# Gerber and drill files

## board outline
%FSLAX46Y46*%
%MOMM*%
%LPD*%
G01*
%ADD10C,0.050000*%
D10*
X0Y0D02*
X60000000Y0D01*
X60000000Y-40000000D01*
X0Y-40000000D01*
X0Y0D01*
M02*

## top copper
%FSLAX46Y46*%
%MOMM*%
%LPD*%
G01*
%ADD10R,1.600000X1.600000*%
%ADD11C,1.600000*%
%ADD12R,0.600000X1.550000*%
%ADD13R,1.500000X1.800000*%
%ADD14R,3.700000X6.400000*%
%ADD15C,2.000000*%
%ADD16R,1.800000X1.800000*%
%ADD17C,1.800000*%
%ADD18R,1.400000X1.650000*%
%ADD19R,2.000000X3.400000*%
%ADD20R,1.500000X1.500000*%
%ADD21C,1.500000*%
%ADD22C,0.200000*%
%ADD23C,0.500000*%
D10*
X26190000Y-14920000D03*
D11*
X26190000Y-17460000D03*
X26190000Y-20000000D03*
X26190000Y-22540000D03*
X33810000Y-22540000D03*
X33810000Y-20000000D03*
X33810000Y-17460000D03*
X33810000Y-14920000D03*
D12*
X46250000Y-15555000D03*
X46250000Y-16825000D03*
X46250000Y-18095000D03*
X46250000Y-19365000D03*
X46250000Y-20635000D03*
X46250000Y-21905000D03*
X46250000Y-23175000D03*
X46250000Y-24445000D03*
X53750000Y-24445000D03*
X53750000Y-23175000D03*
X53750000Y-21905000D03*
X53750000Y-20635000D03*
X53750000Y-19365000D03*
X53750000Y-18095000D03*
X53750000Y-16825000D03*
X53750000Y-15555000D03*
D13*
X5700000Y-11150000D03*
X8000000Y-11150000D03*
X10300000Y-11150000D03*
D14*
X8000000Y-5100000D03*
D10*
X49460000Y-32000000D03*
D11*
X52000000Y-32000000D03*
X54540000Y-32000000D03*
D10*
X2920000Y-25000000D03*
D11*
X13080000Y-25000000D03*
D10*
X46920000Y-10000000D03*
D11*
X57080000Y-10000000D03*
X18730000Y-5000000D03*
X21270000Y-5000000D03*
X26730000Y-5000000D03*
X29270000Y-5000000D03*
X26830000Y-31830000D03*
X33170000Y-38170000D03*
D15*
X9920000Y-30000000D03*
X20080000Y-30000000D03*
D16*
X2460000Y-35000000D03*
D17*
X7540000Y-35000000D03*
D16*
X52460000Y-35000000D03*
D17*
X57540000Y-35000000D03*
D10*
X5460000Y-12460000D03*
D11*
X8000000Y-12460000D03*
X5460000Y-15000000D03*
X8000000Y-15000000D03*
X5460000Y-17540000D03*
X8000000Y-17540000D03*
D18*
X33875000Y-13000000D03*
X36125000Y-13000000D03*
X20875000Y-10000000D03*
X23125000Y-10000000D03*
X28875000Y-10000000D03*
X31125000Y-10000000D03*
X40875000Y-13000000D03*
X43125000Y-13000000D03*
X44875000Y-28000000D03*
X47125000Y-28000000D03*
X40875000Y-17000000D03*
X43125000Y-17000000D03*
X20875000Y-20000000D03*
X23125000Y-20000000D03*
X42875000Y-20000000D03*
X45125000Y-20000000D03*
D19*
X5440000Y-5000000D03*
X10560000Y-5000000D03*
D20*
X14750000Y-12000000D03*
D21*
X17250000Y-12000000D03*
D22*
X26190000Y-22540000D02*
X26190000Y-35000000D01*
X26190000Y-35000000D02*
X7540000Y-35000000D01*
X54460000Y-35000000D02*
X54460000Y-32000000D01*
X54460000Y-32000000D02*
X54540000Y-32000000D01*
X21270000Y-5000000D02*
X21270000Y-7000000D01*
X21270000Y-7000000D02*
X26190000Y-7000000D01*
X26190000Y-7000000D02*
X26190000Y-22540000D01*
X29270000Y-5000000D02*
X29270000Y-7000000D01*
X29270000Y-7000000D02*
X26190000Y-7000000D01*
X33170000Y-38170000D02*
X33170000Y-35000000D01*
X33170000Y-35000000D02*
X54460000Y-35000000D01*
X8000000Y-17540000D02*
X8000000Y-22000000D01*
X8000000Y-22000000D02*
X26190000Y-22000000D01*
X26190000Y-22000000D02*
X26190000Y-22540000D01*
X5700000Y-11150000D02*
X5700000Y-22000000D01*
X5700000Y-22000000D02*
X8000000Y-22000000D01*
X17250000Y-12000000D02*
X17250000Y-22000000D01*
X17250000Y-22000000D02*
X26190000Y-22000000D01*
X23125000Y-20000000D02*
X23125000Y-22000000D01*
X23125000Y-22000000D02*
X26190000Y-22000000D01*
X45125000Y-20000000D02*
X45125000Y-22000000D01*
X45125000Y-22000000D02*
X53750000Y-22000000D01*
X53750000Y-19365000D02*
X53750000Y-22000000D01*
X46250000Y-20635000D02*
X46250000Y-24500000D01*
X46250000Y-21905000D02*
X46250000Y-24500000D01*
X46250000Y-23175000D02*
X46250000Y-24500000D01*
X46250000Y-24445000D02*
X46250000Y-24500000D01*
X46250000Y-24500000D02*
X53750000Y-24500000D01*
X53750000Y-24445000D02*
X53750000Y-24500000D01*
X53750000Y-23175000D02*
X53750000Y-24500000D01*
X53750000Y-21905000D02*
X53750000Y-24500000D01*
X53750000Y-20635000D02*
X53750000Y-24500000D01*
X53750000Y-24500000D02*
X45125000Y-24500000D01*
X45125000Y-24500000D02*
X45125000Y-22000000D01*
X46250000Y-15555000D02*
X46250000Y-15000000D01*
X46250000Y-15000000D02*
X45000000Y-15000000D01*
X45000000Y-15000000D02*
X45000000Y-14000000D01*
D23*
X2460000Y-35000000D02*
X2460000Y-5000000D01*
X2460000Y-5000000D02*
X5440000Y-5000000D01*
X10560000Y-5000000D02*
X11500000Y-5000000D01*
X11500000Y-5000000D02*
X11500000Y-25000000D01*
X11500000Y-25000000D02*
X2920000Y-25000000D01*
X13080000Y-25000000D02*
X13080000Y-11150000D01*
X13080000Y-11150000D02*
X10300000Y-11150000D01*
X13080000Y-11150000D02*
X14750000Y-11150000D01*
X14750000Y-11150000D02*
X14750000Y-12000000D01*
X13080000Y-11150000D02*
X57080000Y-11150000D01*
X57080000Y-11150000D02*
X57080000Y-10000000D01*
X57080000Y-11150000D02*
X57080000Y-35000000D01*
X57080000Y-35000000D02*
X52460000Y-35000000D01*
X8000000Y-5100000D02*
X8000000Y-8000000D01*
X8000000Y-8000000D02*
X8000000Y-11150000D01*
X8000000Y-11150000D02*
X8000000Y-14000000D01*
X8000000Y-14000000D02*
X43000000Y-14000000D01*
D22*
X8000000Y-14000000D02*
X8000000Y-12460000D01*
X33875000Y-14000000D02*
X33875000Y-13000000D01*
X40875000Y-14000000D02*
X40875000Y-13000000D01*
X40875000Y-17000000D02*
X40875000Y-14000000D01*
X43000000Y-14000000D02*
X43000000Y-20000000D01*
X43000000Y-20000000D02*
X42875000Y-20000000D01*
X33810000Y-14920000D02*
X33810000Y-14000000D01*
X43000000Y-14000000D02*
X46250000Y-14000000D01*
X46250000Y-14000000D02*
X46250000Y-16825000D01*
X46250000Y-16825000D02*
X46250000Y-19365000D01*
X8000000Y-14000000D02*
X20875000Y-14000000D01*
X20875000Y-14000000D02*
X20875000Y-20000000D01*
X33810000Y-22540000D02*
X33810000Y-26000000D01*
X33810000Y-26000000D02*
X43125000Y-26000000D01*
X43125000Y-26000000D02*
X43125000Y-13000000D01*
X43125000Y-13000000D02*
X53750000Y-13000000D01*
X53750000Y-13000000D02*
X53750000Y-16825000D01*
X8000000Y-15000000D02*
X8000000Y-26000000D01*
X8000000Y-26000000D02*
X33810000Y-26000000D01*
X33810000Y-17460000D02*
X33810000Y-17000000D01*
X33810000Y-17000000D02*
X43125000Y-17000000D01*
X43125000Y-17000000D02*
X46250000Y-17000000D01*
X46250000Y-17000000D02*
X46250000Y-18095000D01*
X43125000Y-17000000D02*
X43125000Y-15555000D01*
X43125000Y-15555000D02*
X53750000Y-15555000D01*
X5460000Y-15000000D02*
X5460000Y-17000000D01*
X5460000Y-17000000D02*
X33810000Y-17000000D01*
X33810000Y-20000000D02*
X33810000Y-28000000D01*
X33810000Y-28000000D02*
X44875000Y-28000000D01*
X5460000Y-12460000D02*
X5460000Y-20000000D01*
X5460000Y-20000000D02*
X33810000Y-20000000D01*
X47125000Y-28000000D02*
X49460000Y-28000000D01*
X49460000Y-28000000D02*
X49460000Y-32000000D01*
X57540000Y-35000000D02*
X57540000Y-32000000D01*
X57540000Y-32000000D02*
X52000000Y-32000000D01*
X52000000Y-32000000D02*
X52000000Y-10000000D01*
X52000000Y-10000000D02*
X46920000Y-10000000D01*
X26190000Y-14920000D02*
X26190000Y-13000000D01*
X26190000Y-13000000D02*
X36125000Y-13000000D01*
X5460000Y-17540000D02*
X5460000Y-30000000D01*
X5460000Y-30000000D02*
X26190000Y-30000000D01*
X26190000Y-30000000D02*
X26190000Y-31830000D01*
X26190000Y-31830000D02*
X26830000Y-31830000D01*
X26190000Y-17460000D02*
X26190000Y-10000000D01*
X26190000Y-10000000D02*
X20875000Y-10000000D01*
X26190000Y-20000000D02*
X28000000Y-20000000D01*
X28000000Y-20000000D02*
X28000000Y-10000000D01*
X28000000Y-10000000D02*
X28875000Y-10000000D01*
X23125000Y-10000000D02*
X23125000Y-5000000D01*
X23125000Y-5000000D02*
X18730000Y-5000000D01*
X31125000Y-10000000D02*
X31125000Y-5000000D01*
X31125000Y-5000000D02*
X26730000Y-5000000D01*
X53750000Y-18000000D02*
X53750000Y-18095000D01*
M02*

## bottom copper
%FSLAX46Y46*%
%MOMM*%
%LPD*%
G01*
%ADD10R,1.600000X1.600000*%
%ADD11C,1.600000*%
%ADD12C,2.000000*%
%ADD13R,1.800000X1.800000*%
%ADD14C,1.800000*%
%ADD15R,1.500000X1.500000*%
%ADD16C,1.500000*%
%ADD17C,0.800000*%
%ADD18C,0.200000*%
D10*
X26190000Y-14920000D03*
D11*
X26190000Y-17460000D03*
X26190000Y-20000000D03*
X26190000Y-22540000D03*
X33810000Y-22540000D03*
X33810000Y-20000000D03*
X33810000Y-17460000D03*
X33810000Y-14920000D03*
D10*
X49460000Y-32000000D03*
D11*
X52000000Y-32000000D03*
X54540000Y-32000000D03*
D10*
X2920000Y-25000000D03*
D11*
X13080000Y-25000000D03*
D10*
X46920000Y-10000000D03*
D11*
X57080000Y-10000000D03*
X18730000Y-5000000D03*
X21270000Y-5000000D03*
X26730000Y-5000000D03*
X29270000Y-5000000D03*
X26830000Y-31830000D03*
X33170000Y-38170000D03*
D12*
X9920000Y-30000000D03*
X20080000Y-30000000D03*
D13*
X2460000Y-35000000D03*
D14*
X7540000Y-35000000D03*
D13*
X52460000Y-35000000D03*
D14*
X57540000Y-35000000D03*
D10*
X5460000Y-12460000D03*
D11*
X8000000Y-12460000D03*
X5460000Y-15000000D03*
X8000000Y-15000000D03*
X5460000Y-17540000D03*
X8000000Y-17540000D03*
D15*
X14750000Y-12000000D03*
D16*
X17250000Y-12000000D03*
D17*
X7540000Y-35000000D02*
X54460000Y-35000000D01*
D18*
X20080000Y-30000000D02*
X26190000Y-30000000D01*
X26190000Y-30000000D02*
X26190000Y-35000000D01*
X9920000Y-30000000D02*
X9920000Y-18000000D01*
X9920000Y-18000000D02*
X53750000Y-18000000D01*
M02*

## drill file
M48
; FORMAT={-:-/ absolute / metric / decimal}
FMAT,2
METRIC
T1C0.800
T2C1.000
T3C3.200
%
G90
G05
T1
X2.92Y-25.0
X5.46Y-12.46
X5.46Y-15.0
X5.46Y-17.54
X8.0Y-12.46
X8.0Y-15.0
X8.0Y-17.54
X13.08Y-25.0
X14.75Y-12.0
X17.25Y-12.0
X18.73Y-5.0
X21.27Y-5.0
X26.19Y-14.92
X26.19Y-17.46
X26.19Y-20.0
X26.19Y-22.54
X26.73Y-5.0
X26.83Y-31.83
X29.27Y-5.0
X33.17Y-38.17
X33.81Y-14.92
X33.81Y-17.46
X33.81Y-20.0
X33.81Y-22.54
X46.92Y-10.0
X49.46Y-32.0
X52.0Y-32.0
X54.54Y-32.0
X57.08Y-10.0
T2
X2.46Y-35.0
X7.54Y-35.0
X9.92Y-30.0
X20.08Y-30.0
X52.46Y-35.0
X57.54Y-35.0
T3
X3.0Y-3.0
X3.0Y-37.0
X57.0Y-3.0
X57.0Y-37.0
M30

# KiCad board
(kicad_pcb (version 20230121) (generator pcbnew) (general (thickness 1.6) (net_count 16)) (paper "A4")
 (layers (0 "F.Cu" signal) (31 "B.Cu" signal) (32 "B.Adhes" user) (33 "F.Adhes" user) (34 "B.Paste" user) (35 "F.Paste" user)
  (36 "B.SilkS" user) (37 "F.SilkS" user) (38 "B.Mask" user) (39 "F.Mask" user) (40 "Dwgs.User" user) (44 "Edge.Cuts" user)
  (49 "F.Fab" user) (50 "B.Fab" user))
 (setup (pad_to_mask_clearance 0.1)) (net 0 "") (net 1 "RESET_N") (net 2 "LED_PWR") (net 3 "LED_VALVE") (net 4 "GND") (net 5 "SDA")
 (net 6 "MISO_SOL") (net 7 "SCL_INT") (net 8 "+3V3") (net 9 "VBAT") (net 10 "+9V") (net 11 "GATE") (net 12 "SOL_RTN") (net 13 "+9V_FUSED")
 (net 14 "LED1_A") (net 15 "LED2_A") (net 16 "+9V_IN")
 (gr_rect (start 0 0) (end 60 40) (stroke (width 0.05) (type solid)) (layer "Edge.Cuts"))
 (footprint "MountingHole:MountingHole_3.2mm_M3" (layer "F.Cu") (at 3 3) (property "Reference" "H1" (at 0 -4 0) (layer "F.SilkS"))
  (pad "" np_thru_hole circle (at 0 0) (size 3.2 3.2) (drill 3.2) (layers "*.Cu" "*.Mask")))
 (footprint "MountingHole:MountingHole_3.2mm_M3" (layer "F.Cu") (at 57 3) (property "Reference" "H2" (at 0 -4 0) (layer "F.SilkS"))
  (pad "" np_thru_hole circle (at 0 0) (size 3.2 3.2) (drill 3.2) (layers "*.Cu" "*.Mask")))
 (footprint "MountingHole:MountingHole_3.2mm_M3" (layer "F.Cu") (at 3 37) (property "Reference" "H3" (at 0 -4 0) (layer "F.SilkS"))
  (pad "" np_thru_hole circle (at 0 0) (size 3.2 3.2) (drill 3.2) (layers "*.Cu" "*.Mask")))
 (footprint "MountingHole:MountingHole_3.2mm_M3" (layer "F.Cu") (at 57 37) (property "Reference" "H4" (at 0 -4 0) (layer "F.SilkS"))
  (pad "" np_thru_hole circle (at 0 0) (size 3.2 3.2) (drill 3.2) (layers "*.Cu" "*.Mask")))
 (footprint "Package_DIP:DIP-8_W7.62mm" (layer "F.Cu") (at 30 20) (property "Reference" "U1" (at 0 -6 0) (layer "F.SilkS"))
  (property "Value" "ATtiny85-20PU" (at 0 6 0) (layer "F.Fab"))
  (pad "1" thru_hole rect (at -3.8100 -5.0800) (size 1.6 1.6) (drill 0.8) (layers "*.Cu" "*.Mask") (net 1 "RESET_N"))
  (pad "2" thru_hole circle (at -3.8100 -2.5400) (size 1.6 1.6) (drill 0.8) (layers "*.Cu" "*.Mask") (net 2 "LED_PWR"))
  (pad "3" thru_hole circle (at -3.8100 0.0000) (size 1.6 1.6) (drill 0.8) (layers "*.Cu" "*.Mask") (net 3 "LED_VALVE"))
  (pad "4" thru_hole circle (at -3.8100 2.5400) (size 1.6 1.6) (drill 0.8) (layers "*.Cu" "*.Mask") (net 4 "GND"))
  (pad "5" thru_hole circle (at 3.8100 2.5400) (size 1.6 1.6) (drill 0.8) (layers "*.Cu" "*.Mask") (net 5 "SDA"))
  (pad "6" thru_hole circle (at 3.8100 0.0000) (size 1.6 1.6) (drill 0.8) (layers "*.Cu" "*.Mask") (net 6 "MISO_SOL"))
  (pad "7" thru_hole circle (at 3.8100 -2.5400) (size 1.6 1.6) (drill 0.8) (layers "*.Cu" "*.Mask") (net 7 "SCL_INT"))
  (pad "8" thru_hole circle (at 3.8100 -5.0800) (size 1.6 1.6) (drill 0.8) (layers "*.Cu" "*.Mask") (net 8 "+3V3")))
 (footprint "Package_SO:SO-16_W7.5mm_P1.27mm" (layer "F.Cu") (at 50 20) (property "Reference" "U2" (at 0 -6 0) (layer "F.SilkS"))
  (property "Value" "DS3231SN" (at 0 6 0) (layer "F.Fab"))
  (pad "1" smd rect (at -3.75 -4.4450) (size 0.6 1.55) (layers "F.Cu" "F.Paste" "F.Mask") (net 4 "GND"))
  (pad "2" smd rect (at -3.75 -3.1750) (size 0.6 1.55) (layers "F.Cu" "F.Paste" "F.Mask") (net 8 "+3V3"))
  (pad "3" smd rect (at -3.75 -1.9050) (size 0.6 1.55) (layers "F.Cu" "F.Paste" "F.Mask") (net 7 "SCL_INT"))
  (pad "4" smd rect (at -3.75 -0.6350) (size 0.6 1.55) (layers "F.Cu" "F.Paste" "F.Mask") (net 8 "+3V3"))
  (pad "5" smd rect (at -3.75 0.6350) (size 0.6 1.55) (layers "F.Cu" "F.Paste" "F.Mask") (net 4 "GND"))
  (pad "6" smd rect (at -3.75 1.9050) (size 0.6 1.55) (layers "F.Cu" "F.Paste" "F.Mask") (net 4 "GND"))
  (pad "7" smd rect (at -3.75 3.1750) (size 0.6 1.55) (layers "F.Cu" "F.Paste" "F.Mask") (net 4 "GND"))
  (pad "8" smd rect (at -3.75 4.4450) (size 0.6 1.55) (layers "F.Cu" "F.Paste" "F.Mask") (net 4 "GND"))
  (pad "9" smd rect (at 3.75 4.4450) (size 0.6 1.55) (layers "F.Cu" "F.Paste" "F.Mask") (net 4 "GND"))
  (pad "10" smd rect (at 3.75 3.1750) (size 0.6 1.55) (layers "F.Cu" "F.Paste" "F.Mask") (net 4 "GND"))
  (pad "11" smd rect (at 3.75 1.9050) (size 0.6 1.55) (layers "F.Cu" "F.Paste" "F.Mask") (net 4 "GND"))
  (pad "12" smd rect (at 3.75 0.6350) (size 0.6 1.55) (layers "F.Cu" "F.Paste" "F.Mask") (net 4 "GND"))
  (pad "13" smd rect (at 3.75 -0.6350) (size 0.6 1.55) (layers "F.Cu" "F.Paste" "F.Mask") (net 4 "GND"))
  (pad "14" smd rect (at 3.75 -1.9050) (size 0.6 1.55) (layers "F.Cu" "F.Paste" "F.Mask") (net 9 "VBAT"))
  (pad "15" smd rect (at 3.75 -3.1750) (size 0.6 1.55) (layers "F.Cu" "F.Paste" "F.Mask") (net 5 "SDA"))
  (pad "16" smd rect (at 3.75 -4.4450) (size 0.6 1.55) (layers "F.Cu" "F.Paste" "F.Mask") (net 7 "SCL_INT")))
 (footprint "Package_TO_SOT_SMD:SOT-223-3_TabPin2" (layer "F.Cu") (at 8 8) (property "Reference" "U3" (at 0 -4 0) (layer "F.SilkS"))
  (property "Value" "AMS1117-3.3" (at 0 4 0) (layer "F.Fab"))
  (pad "1" smd rect (at -2.3000 3.1500) (size 1.5 1.8) (layers "F.Cu" "F.Paste" "F.Mask") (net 4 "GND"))
  (pad "2" smd rect (at 0.0000 3.1500) (size 1.5 1.8) (layers "F.Cu" "F.Paste" "F.Mask") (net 8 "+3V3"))
  (pad "3" smd rect (at 2.3000 3.1500) (size 1.5 1.8) (layers "F.Cu" "F.Paste" "F.Mask") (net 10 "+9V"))
  (pad "4" smd rect (at 0 -2.9) (size 3.7 6.4) (layers "F.Cu" "F.Paste" "F.Mask") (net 8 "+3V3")))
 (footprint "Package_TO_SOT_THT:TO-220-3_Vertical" (layer "F.Cu") (at 52 32) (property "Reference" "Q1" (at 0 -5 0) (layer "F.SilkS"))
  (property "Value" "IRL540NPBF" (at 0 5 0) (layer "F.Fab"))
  (pad "1" thru_hole rect (at -2.5400 0) (size 1.6 1.6) (drill 0.8) (layers "*.Cu" "*.Mask") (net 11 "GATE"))
  (pad "2" thru_hole circle (at 0.0000 0) (size 1.6 1.6) (drill 0.8) (layers "*.Cu" "*.Mask") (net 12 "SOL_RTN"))
  (pad "3" thru_hole circle (at 2.5400 0) (size 1.6 1.6) (drill 0.8) (layers "*.Cu" "*.Mask") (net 4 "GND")))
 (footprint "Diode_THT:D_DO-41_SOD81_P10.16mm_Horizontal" (layer "F.Cu") (at 8 25) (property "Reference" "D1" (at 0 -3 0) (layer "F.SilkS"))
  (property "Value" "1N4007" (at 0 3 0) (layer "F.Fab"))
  (pad "A" thru_hole rect (at -5.0800 0) (size 1.6 1.6) (drill 0.8) (layers "*.Cu" "*.Mask") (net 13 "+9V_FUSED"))
  (pad "K" thru_hole circle (at 5.0800 0) (size 1.6 1.6) (drill 0.8) (layers "*.Cu" "*.Mask") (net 10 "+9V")))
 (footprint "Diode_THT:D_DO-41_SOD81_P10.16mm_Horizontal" (layer "F.Cu") (at 52 10)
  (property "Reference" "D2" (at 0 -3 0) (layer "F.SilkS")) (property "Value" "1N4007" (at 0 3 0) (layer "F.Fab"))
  (pad "A" thru_hole rect (at -5.0800 0) (size 1.6 1.6) (drill 0.8) (layers "*.Cu" "*.Mask") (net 12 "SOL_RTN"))
  (pad "K" thru_hole circle (at 5.0800 0) (size 1.6 1.6) (drill 0.8) (layers "*.Cu" "*.Mask") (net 10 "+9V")))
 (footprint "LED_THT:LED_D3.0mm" (layer "F.Cu") (at 20 5) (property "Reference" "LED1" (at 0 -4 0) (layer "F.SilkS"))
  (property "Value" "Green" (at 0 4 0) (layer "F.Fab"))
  (pad "A" thru_hole circle (at -1.2700 0) (size 1.6 1.6) (drill 0.8) (layers "*.Cu" "*.Mask") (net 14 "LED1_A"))
  (pad "K" thru_hole circle (at 1.2700 0) (size 1.6 1.6) (drill 0.8) (layers "*.Cu" "*.Mask") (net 4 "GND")))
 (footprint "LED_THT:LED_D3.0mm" (layer "F.Cu") (at 28 5) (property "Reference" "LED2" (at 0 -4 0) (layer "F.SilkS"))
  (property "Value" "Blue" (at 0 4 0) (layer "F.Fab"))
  (pad "A" thru_hole circle (at -1.2700 0) (size 1.6 1.6) (drill 0.8) (layers "*.Cu" "*.Mask") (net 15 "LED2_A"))
  (pad "K" thru_hole circle (at 1.2700 0) (size 1.6 1.6) (drill 0.8) (layers "*.Cu" "*.Mask") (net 4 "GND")))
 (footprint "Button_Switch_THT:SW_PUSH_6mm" (layer "F.Cu") (at 30 35) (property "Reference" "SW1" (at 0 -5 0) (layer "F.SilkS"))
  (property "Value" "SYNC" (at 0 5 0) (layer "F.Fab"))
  (pad "1" thru_hole circle (at -3.1700 -3.1700) (size 1.6 1.6) (drill 0.8) (layers "*.Cu" "*.Mask") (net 1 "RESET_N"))
  (pad "2" thru_hole circle (at 3.1700 3.1700) (size 1.6 1.6) (drill 0.8) (layers "*.Cu" "*.Mask") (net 4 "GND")))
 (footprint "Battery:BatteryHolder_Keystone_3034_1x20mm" (layer "B.Cu") (at 15 30)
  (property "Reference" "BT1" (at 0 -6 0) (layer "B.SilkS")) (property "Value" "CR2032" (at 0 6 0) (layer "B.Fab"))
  (pad "+" thru_hole circle (at -5.0800 0) (size 2 2) (drill 1) (layers "*.Cu" "*.Mask") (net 9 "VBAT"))
  (pad "-" thru_hole circle (at 5.0800 0) (size 2 2) (drill 1) (layers "*.Cu" "*.Mask") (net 4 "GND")))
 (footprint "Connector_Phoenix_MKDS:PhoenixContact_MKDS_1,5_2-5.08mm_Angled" (layer "F.Cu") (at 5 35)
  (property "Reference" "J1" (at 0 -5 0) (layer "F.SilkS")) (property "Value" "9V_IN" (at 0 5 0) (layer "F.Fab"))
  (pad "1" thru_hole rect (at -2.5400 0) (size 1.8 1.8) (drill 1) (layers "*.Cu" "*.Mask") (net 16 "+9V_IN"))
  (pad "2" thru_hole circle (at 2.5400 0) (size 1.8 1.8) (drill 1) (layers "*.Cu" "*.Mask") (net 4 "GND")))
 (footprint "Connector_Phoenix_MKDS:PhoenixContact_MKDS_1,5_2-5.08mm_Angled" (layer "F.Cu") (at 55 35)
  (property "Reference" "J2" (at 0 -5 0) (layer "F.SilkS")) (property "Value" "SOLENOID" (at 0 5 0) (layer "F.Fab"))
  (pad "1" thru_hole rect (at -2.5400 0) (size 1.8 1.8) (drill 1) (layers "*.Cu" "*.Mask") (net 10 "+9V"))
  (pad "2" thru_hole circle (at 2.5400 0) (size 1.8 1.8) (drill 1) (layers "*.Cu" "*.Mask") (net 12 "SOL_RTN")))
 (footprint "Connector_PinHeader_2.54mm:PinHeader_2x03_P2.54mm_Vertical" (layer "F.Cu") (at 8 15)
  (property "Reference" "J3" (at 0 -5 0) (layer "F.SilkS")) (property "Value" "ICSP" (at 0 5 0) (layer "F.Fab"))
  (pad "1" thru_hole rect (at -2.5400 -2.5400) (size 1.6 1.6) (drill 0.8) (layers "*.Cu" "*.Mask") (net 6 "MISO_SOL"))
  (pad "2" thru_hole circle (at 0.0000 -2.5400) (size 1.6 1.6) (drill 0.8) (layers "*.Cu" "*.Mask") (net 8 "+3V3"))
  (pad "3" thru_hole circle (at -2.5400 0.0000) (size 1.6 1.6) (drill 0.8) (layers "*.Cu" "*.Mask") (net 7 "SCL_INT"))
  (pad "4" thru_hole circle (at 0.0000 0.0000) (size 1.6 1.6) (drill 0.8) (layers "*.Cu" "*.Mask") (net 5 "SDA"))
  (pad "5" thru_hole circle (at -2.5400 2.5400) (size 1.6 1.6) (drill 0.8) (layers "*.Cu" "*.Mask") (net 1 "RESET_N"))
  (pad "6" thru_hole circle (at 0.0000 2.5400) (size 1.6 1.6) (drill 0.8) (layers "*.Cu" "*.Mask") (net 4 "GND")))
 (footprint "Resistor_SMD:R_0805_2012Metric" (layer "F.Cu") (at 35 13) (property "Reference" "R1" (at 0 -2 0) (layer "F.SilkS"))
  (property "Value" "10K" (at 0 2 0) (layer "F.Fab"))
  (pad "1" smd rect (at -1.1250 0) (size 1.4 1.65) (layers "F.Cu" "F.Paste" "F.Mask") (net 8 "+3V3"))
  (pad "2" smd rect (at 1.1250 0) (size 1.4 1.65) (layers "F.Cu" "F.Paste" "F.Mask") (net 1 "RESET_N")))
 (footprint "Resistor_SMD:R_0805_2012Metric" (layer "F.Cu") (at 22 10) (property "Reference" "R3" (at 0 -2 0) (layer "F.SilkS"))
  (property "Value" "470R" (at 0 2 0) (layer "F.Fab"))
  (pad "1" smd rect (at -1.1250 0) (size 1.4 1.65) (layers "F.Cu" "F.Paste" "F.Mask") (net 2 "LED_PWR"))
  (pad "2" smd rect (at 1.1250 0) (size 1.4 1.65) (layers "F.Cu" "F.Paste" "F.Mask") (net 14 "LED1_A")))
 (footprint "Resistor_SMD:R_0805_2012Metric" (layer "F.Cu") (at 30 10) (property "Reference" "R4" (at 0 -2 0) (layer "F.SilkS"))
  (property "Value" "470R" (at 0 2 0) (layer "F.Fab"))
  (pad "1" smd rect (at -1.1250 0) (size 1.4 1.65) (layers "F.Cu" "F.Paste" "F.Mask") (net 3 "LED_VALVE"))
  (pad "2" smd rect (at 1.1250 0) (size 1.4 1.65) (layers "F.Cu" "F.Paste" "F.Mask") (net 15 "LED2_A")))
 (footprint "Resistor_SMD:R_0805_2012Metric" (layer "F.Cu") (at 42 13) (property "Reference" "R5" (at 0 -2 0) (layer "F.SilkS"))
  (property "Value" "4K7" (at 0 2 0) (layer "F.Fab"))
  (pad "1" smd rect (at -1.1250 0) (size 1.4 1.65) (layers "F.Cu" "F.Paste" "F.Mask") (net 8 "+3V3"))
  (pad "2" smd rect (at 1.1250 0) (size 1.4 1.65) (layers "F.Cu" "F.Paste" "F.Mask") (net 5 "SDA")))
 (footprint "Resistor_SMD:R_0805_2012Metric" (layer "F.Cu") (at 46 28) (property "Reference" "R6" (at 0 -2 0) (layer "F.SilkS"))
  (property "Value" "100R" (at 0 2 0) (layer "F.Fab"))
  (pad "1" smd rect (at -1.1250 0) (size 1.4 1.65) (layers "F.Cu" "F.Paste" "F.Mask") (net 6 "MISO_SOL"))
  (pad "2" smd rect (at 1.1250 0) (size 1.4 1.65) (layers "F.Cu" "F.Paste" "F.Mask") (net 11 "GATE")))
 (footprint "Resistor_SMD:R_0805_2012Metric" (layer "F.Cu") (at 42 17) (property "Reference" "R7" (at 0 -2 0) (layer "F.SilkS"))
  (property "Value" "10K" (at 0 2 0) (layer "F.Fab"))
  (pad "1" smd rect (at -1.1250 0) (size 1.4 1.65) (layers "F.Cu" "F.Paste" "F.Mask") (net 8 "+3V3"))
  (pad "2" smd rect (at 1.1250 0) (size 1.4 1.65) (layers "F.Cu" "F.Paste" "F.Mask") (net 7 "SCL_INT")))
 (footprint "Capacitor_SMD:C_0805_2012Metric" (layer "F.Cu") (at 22 20) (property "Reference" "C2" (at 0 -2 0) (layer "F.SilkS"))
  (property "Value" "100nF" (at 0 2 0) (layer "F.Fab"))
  (pad "1" smd rect (at -1.1250 0) (size 1.4 1.65) (layers "F.Cu" "F.Paste" "F.Mask") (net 8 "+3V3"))
  (pad "2" smd rect (at 1.1250 0) (size 1.4 1.65) (layers "F.Cu" "F.Paste" "F.Mask") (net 4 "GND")))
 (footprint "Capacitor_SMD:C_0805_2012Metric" (layer "F.Cu") (at 44 20) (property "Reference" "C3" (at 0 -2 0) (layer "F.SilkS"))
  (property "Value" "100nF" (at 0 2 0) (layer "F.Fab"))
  (pad "1" smd rect (at -1.1250 0) (size 1.4 1.65) (layers "F.Cu" "F.Paste" "F.Mask") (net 8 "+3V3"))
  (pad "2" smd rect (at 1.1250 0) (size 1.4 1.65) (layers "F.Cu" "F.Paste" "F.Mask") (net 4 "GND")))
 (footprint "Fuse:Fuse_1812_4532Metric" (layer "F.Cu") (at 8 5) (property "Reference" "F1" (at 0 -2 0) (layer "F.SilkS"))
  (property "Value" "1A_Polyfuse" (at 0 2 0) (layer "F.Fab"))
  (pad "1" smd rect (at -2.5600 0) (size 2.0 3.4) (layers "F.Cu" "F.Paste" "F.Mask") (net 16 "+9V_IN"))
  (pad "2" smd rect (at 2.5600 0) (size 2.0 3.4) (layers "F.Cu" "F.Paste" "F.Mask") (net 13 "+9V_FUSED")))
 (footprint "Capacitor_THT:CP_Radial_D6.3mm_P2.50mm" (layer "F.Cu") (at 16 12) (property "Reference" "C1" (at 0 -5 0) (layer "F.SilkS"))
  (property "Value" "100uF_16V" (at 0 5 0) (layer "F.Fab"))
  (pad "1" thru_hole rect (at -1.2500 0) (size 1.5 1.5) (drill 0.8) (layers "*.Cu" "*.Mask") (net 10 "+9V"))
  (pad "2" thru_hole circle (at 1.2500 0) (size 1.5 1.5) (drill 0.8) (layers "*.Cu" "*.Mask") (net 4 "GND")))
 (segment (start 7.5400 35.0000) (end 54.4600 35.0000) (width 0.8) (layer "B.Cu") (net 4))
 (segment (start 26.1900 22.5400) (end 26.1900 35.0000) (width 0.2) (layer "F.Cu") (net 4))
 (segment (start 26.1900 35.0000) (end 7.5400 35.0000) (width 0.2) (layer "F.Cu") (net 4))
 (segment (start 54.4600 35.0000) (end 54.4600 32.0000) (width 0.2) (layer "F.Cu") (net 4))
 (segment (start 54.4600 32.0000) (end 54.5400 32.0000) (width 0.2) (layer "F.Cu") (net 4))
 (segment (start 21.2700 5.0000) (end 21.2700 7.0000) (width 0.2) (layer "F.Cu") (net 4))
 (segment (start 21.2700 7.0000) (end 26.1900 7.0000) (width 0.2) (layer "F.Cu") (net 4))
 (segment (start 26.1900 7.0000) (end 26.1900 22.5400) (width 0.2) (layer "F.Cu") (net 4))
 (segment (start 29.2700 5.0000) (end 29.2700 7.0000) (width 0.2) (layer "F.Cu") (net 4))
 (segment (start 29.2700 7.0000) (end 26.1900 7.0000) (width 0.2) (layer "F.Cu") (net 4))
 (segment (start 33.1700 38.1700) (end 33.1700 35.0000) (width 0.2) (layer "F.Cu") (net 4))
 (segment (start 33.1700 35.0000) (end 54.4600 35.0000) (width 0.2) (layer "F.Cu") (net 4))
 (segment (start 8.0000 17.5400) (end 8.0000 22.0000) (width 0.2) (layer "F.Cu") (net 4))
 (segment (start 8.0000 22.0000) (end 26.1900 22.0000) (width 0.2) (layer "F.Cu") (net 4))
 (segment (start 26.1900 22.0000) (end 26.1900 22.5400) (width 0.2) (layer "F.Cu") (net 4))
 (segment (start 5.7000 11.1500) (end 5.7000 22.0000) (width 0.2) (layer "F.Cu") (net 4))
 (segment (start 5.7000 22.0000) (end 8.0000 22.0000) (width 0.2) (layer "F.Cu") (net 4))
 (segment (start 17.2500 12.0000) (end 17.2500 22.0000) (width 0.2) (layer "F.Cu") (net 4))
 (segment (start 17.2500 22.0000) (end 26.1900 22.0000) (width 0.2) (layer "F.Cu") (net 4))
 (segment (start 23.1250 20.0000) (end 23.1250 22.0000) (width 0.2) (layer "F.Cu") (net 4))
 (segment (start 23.1250 22.0000) (end 26.1900 22.0000) (width 0.2) (layer "F.Cu") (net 4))
 (segment (start 45.1250 20.0000) (end 45.1250 22.0000) (width 0.2) (layer "F.Cu") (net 4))
 (segment (start 45.1250 22.0000) (end 53.7500 22.0000) (width 0.2) (layer "F.Cu") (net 4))
 (segment (start 53.7500 19.3650) (end 53.7500 22.0000) (width 0.2) (layer "F.Cu") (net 4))
 (segment (start 46.2500 20.6350) (end 46.2500 24.5000) (width 0.2) (layer "F.Cu") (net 4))
 (segment (start 46.2500 21.9050) (end 46.2500 24.5000) (width 0.2) (layer "F.Cu") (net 4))
 (segment (start 46.2500 23.1750) (end 46.2500 24.5000) (width 0.2) (layer "F.Cu") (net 4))
 (segment (start 46.2500 24.4450) (end 46.2500 24.5000) (width 0.2) (layer "F.Cu") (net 4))
 (segment (start 46.2500 24.5000) (end 53.7500 24.5000) (width 0.2) (layer "F.Cu") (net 4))
 (segment (start 53.7500 24.4450) (end 53.7500 24.5000) (width 0.2) (layer "F.Cu") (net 4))
 (segment (start 53.7500 23.1750) (end 53.7500 24.5000) (width 0.2) (layer "F.Cu") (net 4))
 (segment (start 53.7500 21.9050) (end 53.7500 24.5000) (width 0.2) (layer "F.Cu") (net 4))
 (segment (start 53.7500 20.6350) (end 53.7500 24.5000) (width 0.2) (layer "F.Cu") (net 4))
 (segment (start 53.7500 24.5000) (end 45.1250 24.5000) (width 0.2) (layer "F.Cu") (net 4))
 (segment (start 45.1250 24.5000) (end 45.1250 22.0000) (width 0.2) (layer "F.Cu") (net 4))
 (segment (start 46.2500 15.5550) (end 46.2500 15.0000) (width 0.2) (layer "F.Cu") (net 4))
 (segment (start 46.2500 15.0000) (end 45.0000 15.0000) (width 0.2) (layer "F.Cu") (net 4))
 (segment (start 45.0000 15.0000) (end 45.0000 14.0000) (width 0.2) (layer "F.Cu") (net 4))
 (segment (start 20.0800 30.0000) (end 26.1900 30.0000) (width 0.2) (layer "B.Cu") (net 4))
 (segment (start 26.1900 30.0000) (end 26.1900 35.0000) (width 0.2) (layer "B.Cu") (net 4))
 (segment (start 2.4600 35.0000) (end 2.4600 5.0000) (width 0.5) (layer "F.Cu") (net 16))
 (segment (start 2.4600 5.0000) (end 5.4400 5.0000) (width 0.5) (layer "F.Cu") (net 16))
 (segment (start 10.5600 5.0000) (end 11.5000 5.0000) (width 0.5) (layer "F.Cu") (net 13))
 (segment (start 11.5000 5.0000) (end 11.5000 25.0000) (width 0.5) (layer "F.Cu") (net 13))
 (segment (start 11.5000 25.0000) (end 2.9200 25.0000) (width 0.5) (layer "F.Cu") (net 13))
 (segment (start 13.0800 25.0000) (end 13.0800 11.1500) (width 0.5) (layer "F.Cu") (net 10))
 (segment (start 13.0800 11.1500) (end 10.3000 11.1500) (width 0.5) (layer "F.Cu") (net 10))
 (segment (start 13.0800 11.1500) (end 14.7500 11.1500) (width 0.5) (layer "F.Cu") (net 10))
 (segment (start 14.7500 11.1500) (end 14.7500 12.0000) (width 0.5) (layer "F.Cu") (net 10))
 (segment (start 13.0800 11.1500) (end 57.0800 11.1500) (width 0.5) (layer "F.Cu") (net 10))
 (segment (start 57.0800 11.1500) (end 57.0800 10.0000) (width 0.5) (layer "F.Cu") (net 10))
 (segment (start 57.0800 11.1500) (end 57.0800 35.0000) (width 0.5) (layer "F.Cu") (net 10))
 (segment (start 57.0800 35.0000) (end 52.4600 35.0000) (width 0.5) (layer "F.Cu") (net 10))
 (segment (start 8.0000 5.1000) (end 8.0000 8.0000) (width 0.5) (layer "F.Cu") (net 8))
 (segment (start 8.0000 8.0000) (end 8.0000 11.1500) (width 0.5) (layer "F.Cu") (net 8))
 (segment (start 8.0000 11.1500) (end 8.0000 14.0000) (width 0.5) (layer "F.Cu") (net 8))
 (segment (start 8.0000 14.0000) (end 43.0000 14.0000) (width 0.5) (layer "F.Cu") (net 8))
 (segment (start 8.0000 14.0000) (end 8.0000 12.4600) (width 0.2) (layer "F.Cu") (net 8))
 (segment (start 33.8750 14.0000) (end 33.8750 13.0000) (width 0.2) (layer "F.Cu") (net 8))
 (segment (start 40.8750 14.0000) (end 40.8750 13.0000) (width 0.2) (layer "F.Cu") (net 8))
 (segment (start 40.8750 17.0000) (end 40.8750 14.0000) (width 0.2) (layer "F.Cu") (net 8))
 (segment (start 43.0000 14.0000) (end 43.0000 20.0000) (width 0.2) (layer "F.Cu") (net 8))
 (segment (start 43.0000 20.0000) (end 42.8750 20.0000) (width 0.2) (layer "F.Cu") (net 8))
 (segment (start 33.8100 14.9200) (end 33.8100 14.0000) (width 0.2) (layer "F.Cu") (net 8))
 (segment (start 43.0000 14.0000) (end 46.2500 14.0000) (width 0.2) (layer "F.Cu") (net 8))
 (segment (start 46.2500 14.0000) (end 46.2500 16.8250) (width 0.2) (layer "F.Cu") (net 8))
 (segment (start 46.2500 16.8250) (end 46.2500 19.3650) (width 0.2) (layer "F.Cu") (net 8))
 (segment (start 8.0000 14.0000) (end 20.8750 14.0000) (width 0.2) (layer "F.Cu") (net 8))
 (segment (start 20.8750 14.0000) (end 20.8750 20.0000) (width 0.2) (layer "F.Cu") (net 8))
 (segment (start 33.8100 22.5400) (end 33.8100 26.0000) (width 0.2) (layer "F.Cu") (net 5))
 (segment (start 33.8100 26.0000) (end 43.1250 26.0000) (width 0.2) (layer "F.Cu") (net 5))
 (segment (start 43.1250 26.0000) (end 43.1250 13.0000) (width 0.2) (layer "F.Cu") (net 5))
 (segment (start 43.1250 13.0000) (end 53.7500 13.0000) (width 0.2) (layer "F.Cu") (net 5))
 (segment (start 53.7500 13.0000) (end 53.7500 16.8250) (width 0.2) (layer "F.Cu") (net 5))
 (segment (start 8.0000 15.0000) (end 8.0000 26.0000) (width 0.2) (layer "F.Cu") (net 5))
 (segment (start 8.0000 26.0000) (end 33.8100 26.0000) (width 0.2) (layer "F.Cu") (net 5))
 (segment (start 33.8100 17.4600) (end 33.8100 17.0000) (width 0.2) (layer "F.Cu") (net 7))
 (segment (start 33.8100 17.0000) (end 43.1250 17.0000) (width 0.2) (layer "F.Cu") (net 7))
 (segment (start 43.1250 17.0000) (end 46.2500 17.0000) (width 0.2) (layer "F.Cu") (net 7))
 (segment (start 46.2500 17.0000) (end 46.2500 18.0950) (width 0.2) (layer "F.Cu") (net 7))
 (segment (start 43.1250 17.0000) (end 43.1250 15.5550) (width 0.2) (layer "F.Cu") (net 7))
 (segment (start 43.1250 15.5550) (end 53.7500 15.5550) (width 0.2) (layer "F.Cu") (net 7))
 (segment (start 5.4600 15.0000) (end 5.4600 17.0000) (width 0.2) (layer "F.Cu") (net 7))
 (segment (start 5.4600 17.0000) (end 33.8100 17.0000) (width 0.2) (layer "F.Cu") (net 7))
 (segment (start 33.8100 20.0000) (end 33.8100 28.0000) (width 0.2) (layer "F.Cu") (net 6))
 (segment (start 33.8100 28.0000) (end 44.8750 28.0000) (width 0.2) (layer "F.Cu") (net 6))
 (segment (start 5.4600 12.4600) (end 5.4600 20.0000) (width 0.2) (layer "F.Cu") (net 6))
 (segment (start 5.4600 20.0000) (end 33.8100 20.0000) (width 0.2) (layer "F.Cu") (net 6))
 (segment (start 47.1250 28.0000) (end 49.4600 28.0000) (width 0.2) (layer "F.Cu") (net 11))
 (segment (start 49.4600 28.0000) (end 49.4600 32.0000) (width 0.2) (layer "F.Cu") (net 11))
 (segment (start 57.5400 35.0000) (end 57.5400 32.0000) (width 0.2) (layer "F.Cu") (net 12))
 (segment (start 57.5400 32.0000) (end 52.0000 32.0000) (width 0.2) (layer "F.Cu") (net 12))
 (segment (start 52.0000 32.0000) (end 52.0000 10.0000) (width 0.2) (layer "F.Cu") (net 12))
 (segment (start 52.0000 10.0000) (end 46.9200 10.0000) (width 0.2) (layer "F.Cu") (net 12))
 (segment (start 26.1900 14.9200) (end 26.1900 13.0000) (width 0.2) (layer "F.Cu") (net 1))
 (segment (start 26.1900 13.0000) (end 36.1250 13.0000) (width 0.2) (layer "F.Cu") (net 1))
 (segment (start 5.4600 17.5400) (end 5.4600 30.0000) (width 0.2) (layer "F.Cu") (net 1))
 (segment (start 5.4600 30.0000) (end 26.1900 30.0000) (width 0.2) (layer "F.Cu") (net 1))
 (segment (start 26.1900 30.0000) (end 26.1900 31.8300) (width 0.2) (layer "F.Cu") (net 1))
 (segment (start 26.1900 31.8300) (end 26.8300 31.8300) (width 0.2) (layer "F.Cu") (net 1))
 (segment (start 26.1900 17.4600) (end 26.1900 10.0000) (width 0.2) (layer "F.Cu") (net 2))
 (segment (start 26.1900 10.0000) (end 20.8750 10.0000) (width 0.2) (layer "F.Cu") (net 2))
 (segment (start 26.1900 20.0000) (end 28.0000 20.0000) (width 0.2) (layer "F.Cu") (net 3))
 (segment (start 28.0000 20.0000) (end 28.0000 10.0000) (width 0.2) (layer "F.Cu") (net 3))
 (segment (start 28.0000 10.0000) (end 28.8750 10.0000) (width 0.2) (layer "F.Cu") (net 3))
 (segment (start 23.1250 10.0000) (end 23.1250 5.0000) (width 0.2) (layer "F.Cu") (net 14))
 (segment (start 23.1250 5.0000) (end 18.7300 5.0000) (width 0.2) (layer "F.Cu") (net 14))
 (segment (start 31.1250 10.0000) (end 31.1250 5.0000) (width 0.2) (layer "F.Cu") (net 15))
 (segment (start 31.1250 5.0000) (end 26.7300 5.0000) (width 0.2) (layer "F.Cu") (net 15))
 (segment (start 9.9200 30.0000) (end 9.9200 18.0000) (width 0.2) (layer "B.Cu") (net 9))
 (segment (start 9.9200 18.0000) (end 53.7500 18.0000) (width 0.2) (layer "B.Cu") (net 9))
 (segment (start 53.7500 18.0000) (end 53.7500 18.0950) (width 0.2) (layer "F.Cu") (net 9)))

